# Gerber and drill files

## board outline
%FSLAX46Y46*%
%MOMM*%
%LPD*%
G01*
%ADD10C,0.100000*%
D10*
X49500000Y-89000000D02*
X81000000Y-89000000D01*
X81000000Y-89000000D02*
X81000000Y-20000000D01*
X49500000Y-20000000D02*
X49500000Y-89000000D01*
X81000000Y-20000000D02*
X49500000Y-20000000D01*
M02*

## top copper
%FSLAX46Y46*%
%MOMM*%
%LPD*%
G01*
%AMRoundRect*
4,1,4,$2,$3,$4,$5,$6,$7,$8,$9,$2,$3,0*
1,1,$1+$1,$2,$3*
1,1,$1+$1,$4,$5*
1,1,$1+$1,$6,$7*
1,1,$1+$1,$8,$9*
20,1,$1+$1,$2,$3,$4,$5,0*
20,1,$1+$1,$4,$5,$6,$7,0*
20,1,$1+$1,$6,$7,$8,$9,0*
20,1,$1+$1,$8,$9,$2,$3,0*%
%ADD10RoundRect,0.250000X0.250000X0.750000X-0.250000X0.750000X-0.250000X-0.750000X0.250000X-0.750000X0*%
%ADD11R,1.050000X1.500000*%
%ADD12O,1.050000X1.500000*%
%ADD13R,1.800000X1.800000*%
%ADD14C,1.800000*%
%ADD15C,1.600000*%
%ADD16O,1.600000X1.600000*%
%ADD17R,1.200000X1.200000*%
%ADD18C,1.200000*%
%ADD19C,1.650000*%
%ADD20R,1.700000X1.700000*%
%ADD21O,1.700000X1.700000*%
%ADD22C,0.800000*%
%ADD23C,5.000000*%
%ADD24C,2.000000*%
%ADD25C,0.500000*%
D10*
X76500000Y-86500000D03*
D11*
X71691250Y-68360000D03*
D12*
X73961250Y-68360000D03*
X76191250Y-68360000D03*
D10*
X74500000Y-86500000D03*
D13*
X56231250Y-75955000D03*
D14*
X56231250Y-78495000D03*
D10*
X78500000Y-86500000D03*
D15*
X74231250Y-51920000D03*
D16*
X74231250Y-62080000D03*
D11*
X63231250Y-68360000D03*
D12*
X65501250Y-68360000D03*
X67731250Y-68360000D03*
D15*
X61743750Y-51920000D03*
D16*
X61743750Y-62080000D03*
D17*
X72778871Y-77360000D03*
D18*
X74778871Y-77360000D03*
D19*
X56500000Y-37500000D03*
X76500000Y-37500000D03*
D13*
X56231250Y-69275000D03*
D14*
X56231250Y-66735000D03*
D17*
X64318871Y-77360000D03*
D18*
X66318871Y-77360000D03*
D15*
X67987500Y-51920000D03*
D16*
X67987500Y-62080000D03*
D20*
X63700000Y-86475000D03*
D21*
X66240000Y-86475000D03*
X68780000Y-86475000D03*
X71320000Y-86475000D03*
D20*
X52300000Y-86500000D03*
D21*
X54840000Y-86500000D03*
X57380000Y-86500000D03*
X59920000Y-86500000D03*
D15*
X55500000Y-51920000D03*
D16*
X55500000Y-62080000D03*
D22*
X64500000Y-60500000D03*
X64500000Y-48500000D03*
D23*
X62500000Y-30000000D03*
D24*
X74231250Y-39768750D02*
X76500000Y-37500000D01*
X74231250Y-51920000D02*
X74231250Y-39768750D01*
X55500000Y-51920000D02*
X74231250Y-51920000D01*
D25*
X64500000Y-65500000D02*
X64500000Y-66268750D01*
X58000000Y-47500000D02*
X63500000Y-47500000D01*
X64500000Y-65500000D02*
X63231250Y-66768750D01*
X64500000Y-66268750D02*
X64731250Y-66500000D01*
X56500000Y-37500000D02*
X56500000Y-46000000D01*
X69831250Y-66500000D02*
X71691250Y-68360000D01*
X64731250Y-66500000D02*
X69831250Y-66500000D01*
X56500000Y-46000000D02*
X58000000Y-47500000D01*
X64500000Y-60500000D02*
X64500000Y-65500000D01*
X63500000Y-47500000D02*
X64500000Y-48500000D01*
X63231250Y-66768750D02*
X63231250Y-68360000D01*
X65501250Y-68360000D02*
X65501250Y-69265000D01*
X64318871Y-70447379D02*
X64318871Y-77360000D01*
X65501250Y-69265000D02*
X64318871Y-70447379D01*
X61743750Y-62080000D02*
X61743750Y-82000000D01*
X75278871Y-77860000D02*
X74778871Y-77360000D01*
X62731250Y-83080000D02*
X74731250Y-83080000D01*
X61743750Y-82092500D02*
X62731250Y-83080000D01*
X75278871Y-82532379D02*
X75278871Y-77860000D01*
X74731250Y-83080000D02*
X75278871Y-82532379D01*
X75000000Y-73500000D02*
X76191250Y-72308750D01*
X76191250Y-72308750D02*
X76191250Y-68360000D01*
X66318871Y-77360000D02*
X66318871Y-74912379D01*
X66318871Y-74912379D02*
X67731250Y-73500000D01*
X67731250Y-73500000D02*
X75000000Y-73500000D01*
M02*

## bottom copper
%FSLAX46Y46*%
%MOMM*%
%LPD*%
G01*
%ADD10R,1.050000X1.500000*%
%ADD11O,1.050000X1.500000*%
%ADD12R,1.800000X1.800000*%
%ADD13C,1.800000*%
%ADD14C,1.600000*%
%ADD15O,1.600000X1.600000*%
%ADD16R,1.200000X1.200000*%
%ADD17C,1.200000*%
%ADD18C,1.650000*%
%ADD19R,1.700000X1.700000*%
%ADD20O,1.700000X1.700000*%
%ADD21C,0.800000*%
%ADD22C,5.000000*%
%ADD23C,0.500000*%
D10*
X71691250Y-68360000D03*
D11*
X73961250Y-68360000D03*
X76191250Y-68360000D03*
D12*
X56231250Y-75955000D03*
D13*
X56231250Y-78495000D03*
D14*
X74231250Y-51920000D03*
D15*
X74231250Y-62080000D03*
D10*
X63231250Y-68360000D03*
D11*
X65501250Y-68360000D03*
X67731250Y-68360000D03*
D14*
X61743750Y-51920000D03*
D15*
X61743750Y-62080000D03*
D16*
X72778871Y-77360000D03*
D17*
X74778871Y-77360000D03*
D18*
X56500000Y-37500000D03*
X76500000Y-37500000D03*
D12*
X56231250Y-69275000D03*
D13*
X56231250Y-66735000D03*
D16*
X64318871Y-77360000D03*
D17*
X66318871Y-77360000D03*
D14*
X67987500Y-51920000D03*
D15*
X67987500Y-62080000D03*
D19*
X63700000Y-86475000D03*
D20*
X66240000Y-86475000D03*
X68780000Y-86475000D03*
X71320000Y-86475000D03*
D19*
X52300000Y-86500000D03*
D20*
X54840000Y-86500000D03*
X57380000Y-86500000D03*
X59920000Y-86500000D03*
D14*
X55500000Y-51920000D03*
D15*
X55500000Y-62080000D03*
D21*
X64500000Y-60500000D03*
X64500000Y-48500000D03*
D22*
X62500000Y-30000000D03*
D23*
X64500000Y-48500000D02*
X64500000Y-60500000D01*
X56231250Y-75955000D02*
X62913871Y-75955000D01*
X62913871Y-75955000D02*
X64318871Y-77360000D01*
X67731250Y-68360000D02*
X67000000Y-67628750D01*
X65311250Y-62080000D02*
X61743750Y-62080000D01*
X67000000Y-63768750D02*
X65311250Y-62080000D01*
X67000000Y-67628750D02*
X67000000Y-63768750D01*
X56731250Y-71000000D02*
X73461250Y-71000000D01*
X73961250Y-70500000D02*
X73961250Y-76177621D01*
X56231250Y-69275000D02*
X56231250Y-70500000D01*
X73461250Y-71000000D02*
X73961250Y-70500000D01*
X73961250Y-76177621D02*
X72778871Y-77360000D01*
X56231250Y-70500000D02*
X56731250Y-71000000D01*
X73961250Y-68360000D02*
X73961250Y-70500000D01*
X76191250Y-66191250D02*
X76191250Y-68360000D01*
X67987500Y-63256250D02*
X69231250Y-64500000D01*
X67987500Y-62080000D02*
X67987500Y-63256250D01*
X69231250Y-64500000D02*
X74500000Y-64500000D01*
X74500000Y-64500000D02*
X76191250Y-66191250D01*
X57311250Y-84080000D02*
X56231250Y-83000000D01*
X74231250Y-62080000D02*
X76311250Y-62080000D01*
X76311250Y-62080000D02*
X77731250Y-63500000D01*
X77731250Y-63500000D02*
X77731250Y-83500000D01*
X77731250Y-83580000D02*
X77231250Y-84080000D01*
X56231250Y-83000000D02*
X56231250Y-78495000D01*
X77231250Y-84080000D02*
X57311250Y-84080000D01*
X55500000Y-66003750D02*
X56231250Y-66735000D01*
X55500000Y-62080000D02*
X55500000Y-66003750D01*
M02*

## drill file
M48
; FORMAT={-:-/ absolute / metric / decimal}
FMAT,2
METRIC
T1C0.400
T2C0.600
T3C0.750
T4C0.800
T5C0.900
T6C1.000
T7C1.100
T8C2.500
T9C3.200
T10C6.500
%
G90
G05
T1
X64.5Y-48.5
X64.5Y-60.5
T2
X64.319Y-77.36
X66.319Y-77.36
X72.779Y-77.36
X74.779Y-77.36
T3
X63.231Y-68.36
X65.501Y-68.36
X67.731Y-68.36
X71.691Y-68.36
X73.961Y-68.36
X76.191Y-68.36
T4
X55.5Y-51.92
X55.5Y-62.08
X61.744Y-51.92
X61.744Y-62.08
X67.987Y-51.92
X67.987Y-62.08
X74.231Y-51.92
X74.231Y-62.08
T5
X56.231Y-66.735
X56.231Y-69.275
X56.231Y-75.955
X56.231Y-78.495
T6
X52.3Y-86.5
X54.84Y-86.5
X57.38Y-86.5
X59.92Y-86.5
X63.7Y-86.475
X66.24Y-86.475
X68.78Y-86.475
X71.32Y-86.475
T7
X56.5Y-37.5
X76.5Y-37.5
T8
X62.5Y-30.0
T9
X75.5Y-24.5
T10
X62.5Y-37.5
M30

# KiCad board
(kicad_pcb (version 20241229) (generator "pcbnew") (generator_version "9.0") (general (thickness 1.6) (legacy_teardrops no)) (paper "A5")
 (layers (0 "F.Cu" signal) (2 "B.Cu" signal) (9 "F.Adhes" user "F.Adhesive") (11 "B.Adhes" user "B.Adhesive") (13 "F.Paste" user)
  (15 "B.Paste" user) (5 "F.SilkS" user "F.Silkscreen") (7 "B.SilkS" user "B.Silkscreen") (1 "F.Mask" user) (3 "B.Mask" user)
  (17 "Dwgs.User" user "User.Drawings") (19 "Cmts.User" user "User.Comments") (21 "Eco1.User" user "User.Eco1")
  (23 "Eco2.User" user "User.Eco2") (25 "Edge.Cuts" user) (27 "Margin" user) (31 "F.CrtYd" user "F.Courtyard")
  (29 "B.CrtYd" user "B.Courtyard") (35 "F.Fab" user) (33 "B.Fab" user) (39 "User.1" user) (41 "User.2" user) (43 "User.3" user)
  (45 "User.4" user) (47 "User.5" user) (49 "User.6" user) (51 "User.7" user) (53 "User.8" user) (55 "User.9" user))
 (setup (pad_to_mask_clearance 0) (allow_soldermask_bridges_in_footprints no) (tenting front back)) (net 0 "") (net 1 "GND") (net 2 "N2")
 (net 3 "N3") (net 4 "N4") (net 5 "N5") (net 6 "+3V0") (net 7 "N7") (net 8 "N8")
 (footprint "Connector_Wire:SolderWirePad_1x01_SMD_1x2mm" (layer "F.Cu") (at 76.5 86.5 180)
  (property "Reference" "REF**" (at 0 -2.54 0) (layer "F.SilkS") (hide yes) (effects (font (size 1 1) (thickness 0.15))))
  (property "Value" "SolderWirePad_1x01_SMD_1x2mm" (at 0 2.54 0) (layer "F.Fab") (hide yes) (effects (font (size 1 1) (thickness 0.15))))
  (pad "1" smd roundrect (at 0 0 180) (size 1 2) (layers "F.Cu" "F.Mask" "F.Paste") (roundrect_rratio 0.25)))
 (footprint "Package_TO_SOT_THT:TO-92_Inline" (layer "F.Cu") (at 72.69125 68.36)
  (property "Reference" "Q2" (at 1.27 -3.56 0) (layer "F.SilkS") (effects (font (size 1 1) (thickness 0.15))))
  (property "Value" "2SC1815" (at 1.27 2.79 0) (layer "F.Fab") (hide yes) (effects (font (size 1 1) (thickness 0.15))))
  (pad "1" thru_hole rect (at -1 0) (size 1.05 1.5) (drill 0.75) (layers "*.Cu" "*.Mask") (remove_unused_layers no) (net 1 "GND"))
  (pad "2" thru_hole oval (at 1.27 0) (size 1.05 1.5) (drill 0.75) (layers "*.Cu" "*.Mask") (remove_unused_layers no) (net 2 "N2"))
  (pad "3" thru_hole oval (at 3.5 0) (size 1.05 1.5) (drill 0.75) (layers "*.Cu" "*.Mask") (remove_unused_layers no) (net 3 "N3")))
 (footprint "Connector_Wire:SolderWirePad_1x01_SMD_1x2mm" (layer "F.Cu") (at 74.5 86.5 180)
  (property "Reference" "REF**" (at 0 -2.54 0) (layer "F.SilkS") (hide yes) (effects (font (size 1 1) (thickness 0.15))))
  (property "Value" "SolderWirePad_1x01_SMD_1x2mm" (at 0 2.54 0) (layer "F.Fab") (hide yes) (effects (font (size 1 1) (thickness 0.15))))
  (pad "1" smd roundrect (at 0 0 180) (size 1 2) (layers "F.Cu" "F.Mask" "F.Paste") (roundrect_rratio 0.25)))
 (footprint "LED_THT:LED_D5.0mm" (layer "F.Cu") (at 56.23125 75.955 -90)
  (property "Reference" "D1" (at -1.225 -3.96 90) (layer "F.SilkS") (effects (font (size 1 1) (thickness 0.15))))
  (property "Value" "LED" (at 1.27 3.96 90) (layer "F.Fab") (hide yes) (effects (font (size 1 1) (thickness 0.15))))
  (pad "1" thru_hole rect (at 0 0 270) (size 1.8 1.8) (drill 0.9) (layers "*.Cu" "*.Mask") (remove_unused_layers no) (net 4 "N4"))
  (pad "2" thru_hole circle (at 2.54 0 270) (size 1.8 1.8) (drill 0.9) (layers "*.Cu" "*.Mask") (remove_unused_layers no) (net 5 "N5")))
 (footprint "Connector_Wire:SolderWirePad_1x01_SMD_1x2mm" (layer "F.Cu") (at 78.5 86.5 180)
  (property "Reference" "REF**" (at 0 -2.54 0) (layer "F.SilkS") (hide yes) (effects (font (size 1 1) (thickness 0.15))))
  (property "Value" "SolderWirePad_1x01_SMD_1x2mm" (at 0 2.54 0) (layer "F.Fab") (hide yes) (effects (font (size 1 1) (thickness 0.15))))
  (pad "1" smd roundrect (at 0 0 180) (size 1 2) (layers "F.Cu" "F.Mask" "F.Paste") (roundrect_rratio 0.25)))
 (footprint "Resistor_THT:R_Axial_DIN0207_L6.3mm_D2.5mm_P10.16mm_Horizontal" (layer "F.Cu") (at 74.23125 51.92 -90)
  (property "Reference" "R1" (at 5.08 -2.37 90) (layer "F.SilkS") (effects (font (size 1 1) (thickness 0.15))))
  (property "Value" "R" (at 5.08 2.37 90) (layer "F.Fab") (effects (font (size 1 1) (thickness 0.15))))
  (pad "1" thru_hole circle (at 0 0 270) (size 1.6 1.6) (drill 0.8) (layers "*.Cu" "*.Mask") (remove_unused_layers no) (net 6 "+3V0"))
  (pad "2" thru_hole oval (at 10.16 0 270) (size 1.6 1.6) (drill 0.8) (layers "*.Cu" "*.Mask") (remove_unused_layers no) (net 5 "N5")))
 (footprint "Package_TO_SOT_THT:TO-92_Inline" (layer "F.Cu") (at 64.23125 68.36)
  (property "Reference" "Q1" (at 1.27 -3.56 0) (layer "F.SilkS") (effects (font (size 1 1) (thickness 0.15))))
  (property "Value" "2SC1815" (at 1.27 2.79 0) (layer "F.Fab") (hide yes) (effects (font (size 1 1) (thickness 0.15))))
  (pad "1" thru_hole rect (at -1 0) (size 1.05 1.5) (drill 0.75) (layers "*.Cu" "*.Mask") (remove_unused_layers no) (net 1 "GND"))
  (pad "2" thru_hole oval (at 1.27 0) (size 1.05 1.5) (drill 0.75) (layers "*.Cu" "*.Mask") (remove_unused_layers no) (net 4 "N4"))
  (pad "3" thru_hole oval (at 3.5 0) (size 1.05 1.5) (drill 0.75) (layers "*.Cu" "*.Mask") (remove_unused_layers no) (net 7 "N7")))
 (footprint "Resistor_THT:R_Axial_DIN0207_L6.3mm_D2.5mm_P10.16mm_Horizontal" (layer "F.Cu") (at 61.74375 51.92 -90)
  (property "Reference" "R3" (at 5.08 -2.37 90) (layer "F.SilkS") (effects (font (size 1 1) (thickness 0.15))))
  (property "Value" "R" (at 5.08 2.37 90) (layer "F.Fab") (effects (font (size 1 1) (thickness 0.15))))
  (pad "1" thru_hole circle (at 0 0 270) (size 1.6 1.6) (drill 0.8) (layers "*.Cu" "*.Mask") (remove_unused_layers no) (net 6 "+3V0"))
  (pad "2" thru_hole oval (at 10.16 0 270) (size 1.6 1.6) (drill 0.8) (layers "*.Cu" "*.Mask") (remove_unused_layers no) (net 7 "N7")))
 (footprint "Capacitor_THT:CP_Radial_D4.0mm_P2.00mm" (layer "F.Cu") (at 72.778871 77.36)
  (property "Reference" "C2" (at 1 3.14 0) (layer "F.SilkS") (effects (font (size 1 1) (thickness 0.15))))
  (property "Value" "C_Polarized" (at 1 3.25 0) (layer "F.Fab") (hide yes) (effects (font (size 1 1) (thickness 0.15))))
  (pad "1" thru_hole rect (at 0 0) (size 1.2 1.2) (drill 0.6) (layers "*.Cu" "*.Mask") (remove_unused_layers no) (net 2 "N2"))
  (pad "2" thru_hole circle (at 2 0) (size 1.2 1.2) (drill 0.6) (layers "*.Cu" "*.Mask") (remove_unused_layers no) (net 7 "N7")))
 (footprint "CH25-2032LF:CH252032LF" (layer "F.Cu") (at 56.5 37.5 90)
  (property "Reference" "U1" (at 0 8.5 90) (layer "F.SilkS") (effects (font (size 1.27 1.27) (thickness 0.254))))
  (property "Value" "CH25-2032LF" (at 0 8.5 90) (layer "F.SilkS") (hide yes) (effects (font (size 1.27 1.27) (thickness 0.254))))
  (pad "" np_thru_hole circle (at 0 6 90) (size 6.5 6.5) (drill 6.5) (layers "*.Cu" "*.Mask"))
  (pad "1" thru_hole circle (at 0 0 90) (size 1.65 1.65) (drill 1.1) (layers "*.Cu" "*.Mask") (remove_unused_layers no) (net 1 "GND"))
  (pad "2" thru_hole circle (at 0 20 90) (size 1.65 1.65) (drill 1.1) (layers "*.Cu" "*.Mask") (remove_unused_layers no) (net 6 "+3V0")))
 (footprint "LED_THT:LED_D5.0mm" (layer "F.Cu") (at 56.23125 69.275 90)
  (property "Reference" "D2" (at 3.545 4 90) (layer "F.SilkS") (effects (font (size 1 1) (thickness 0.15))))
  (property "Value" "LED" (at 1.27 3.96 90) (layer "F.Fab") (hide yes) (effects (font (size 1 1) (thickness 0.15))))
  (pad "1" thru_hole rect (at 0 0 90) (size 1.8 1.8) (drill 0.9) (layers "*.Cu" "*.Mask") (remove_unused_layers no) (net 2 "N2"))
  (pad "2" thru_hole circle (at 2.54 0 90) (size 1.8 1.8) (drill 0.9) (layers "*.Cu" "*.Mask") (remove_unused_layers no) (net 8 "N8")))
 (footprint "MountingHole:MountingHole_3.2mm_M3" (layer "F.Cu") (at 75.5 24.5)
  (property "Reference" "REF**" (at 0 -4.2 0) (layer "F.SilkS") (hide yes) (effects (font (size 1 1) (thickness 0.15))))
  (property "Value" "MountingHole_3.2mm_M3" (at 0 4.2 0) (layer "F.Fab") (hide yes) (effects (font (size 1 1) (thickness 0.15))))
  (pad "" np_thru_hole circle (at 0 0) (size 3.2 3.2) (drill 3.2) (layers "*.Cu" "*.Mask")))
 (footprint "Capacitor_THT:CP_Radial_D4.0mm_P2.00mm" (layer "F.Cu") (at 64.318871 77.36)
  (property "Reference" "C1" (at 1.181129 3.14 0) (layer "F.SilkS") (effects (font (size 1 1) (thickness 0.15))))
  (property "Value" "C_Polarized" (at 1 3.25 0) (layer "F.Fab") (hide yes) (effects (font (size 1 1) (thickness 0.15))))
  (pad "1" thru_hole rect (at 0 0) (size 1.2 1.2) (drill 0.6) (layers "*.Cu" "*.Mask") (remove_unused_layers no) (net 4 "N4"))
  (pad "2" thru_hole circle (at 2 0) (size 1.2 1.2) (drill 0.6) (layers "*.Cu" "*.Mask") (remove_unused_layers no) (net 3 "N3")))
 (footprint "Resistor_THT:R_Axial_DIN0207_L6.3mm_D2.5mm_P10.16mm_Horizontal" (layer "F.Cu") (at 67.9875 51.92 -90)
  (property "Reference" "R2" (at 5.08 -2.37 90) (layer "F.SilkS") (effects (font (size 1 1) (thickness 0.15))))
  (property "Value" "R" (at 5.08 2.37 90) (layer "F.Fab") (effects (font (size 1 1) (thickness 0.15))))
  (pad "1" thru_hole circle (at 0 0 270) (size 1.6 1.6) (drill 0.8) (layers "*.Cu" "*.Mask") (remove_unused_layers no) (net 6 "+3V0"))
  (pad "2" thru_hole oval (at 10.16 0 270) (size 1.6 1.6) (drill 0.8) (layers "*.Cu" "*.Mask") (remove_unused_layers no) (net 3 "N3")))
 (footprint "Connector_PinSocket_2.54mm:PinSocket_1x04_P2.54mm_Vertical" (layer "F.Cu") (at 63.7 86.475 90)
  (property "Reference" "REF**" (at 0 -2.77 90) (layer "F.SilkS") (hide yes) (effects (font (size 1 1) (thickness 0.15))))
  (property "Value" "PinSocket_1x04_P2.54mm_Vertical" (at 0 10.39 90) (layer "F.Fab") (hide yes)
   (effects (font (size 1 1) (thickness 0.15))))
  (pad "1" thru_hole rect (at 0 0 90) (size 1.7 1.7) (drill 1) (layers "*.Cu" "*.Mask") (remove_unused_layers no))
  (pad "2" thru_hole oval (at 0 2.54 90) (size 1.7 1.7) (drill 1) (layers "*.Cu" "*.Mask") (remove_unused_layers no))
  (pad "3" thru_hole oval (at 0 5.08 90) (size 1.7 1.7) (drill 1) (layers "*.Cu" "*.Mask") (remove_unused_layers no))
  (pad "4" thru_hole oval (at 0 7.62 90) (size 1.7 1.7) (drill 1) (layers "*.Cu" "*.Mask") (remove_unused_layers no)))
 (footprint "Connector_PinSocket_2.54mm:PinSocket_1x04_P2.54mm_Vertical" (layer "F.Cu") (at 52.3 86.5 90)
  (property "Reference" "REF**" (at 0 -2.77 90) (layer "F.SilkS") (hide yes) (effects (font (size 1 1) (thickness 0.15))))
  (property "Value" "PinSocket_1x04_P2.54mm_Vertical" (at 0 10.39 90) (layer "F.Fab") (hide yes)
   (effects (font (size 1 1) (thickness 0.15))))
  (pad "1" thru_hole rect (at 0 0 90) (size 1.7 1.7) (drill 1) (layers "*.Cu" "*.Mask") (remove_unused_layers no))
  (pad "2" thru_hole oval (at 0 2.54 90) (size 1.7 1.7) (drill 1) (layers "*.Cu" "*.Mask") (remove_unused_layers no))
  (pad "3" thru_hole oval (at 0 5.08 90) (size 1.7 1.7) (drill 1) (layers "*.Cu" "*.Mask") (remove_unused_layers no))
  (pad "4" thru_hole oval (at 0 7.62 90) (size 1.7 1.7) (drill 1) (layers "*.Cu" "*.Mask") (remove_unused_layers no)))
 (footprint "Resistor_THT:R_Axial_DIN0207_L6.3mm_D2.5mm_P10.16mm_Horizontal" (layer "F.Cu") (at 55.5 51.92 -90)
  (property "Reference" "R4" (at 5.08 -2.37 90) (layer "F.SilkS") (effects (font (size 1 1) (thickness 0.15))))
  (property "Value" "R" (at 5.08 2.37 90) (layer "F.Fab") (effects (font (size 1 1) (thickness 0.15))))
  (pad "1" thru_hole circle (at 0 0 270) (size 1.6 1.6) (drill 0.8) (layers "*.Cu" "*.Mask") (remove_unused_layers no) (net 6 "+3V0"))
  (pad "2" thru_hole oval (at 10.16 0 270) (size 1.6 1.6) (drill 0.8) (layers "*.Cu" "*.Mask") (remove_unused_layers no) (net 8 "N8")))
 (gr_line (start 49.5 89) (end 81 89) (stroke (width 0.1) (type default)) (layer "Edge.Cuts"))
 (gr_line (start 81 89) (end 81 20) (stroke (width 0.1) (type default)) (layer "Edge.Cuts"))
 (gr_line (start 49.5 20) (end 49.5 89) (stroke (width 0.1) (type default)) (layer "Edge.Cuts"))
 (gr_line (start 81 20) (end 49.5 20) (stroke (width 0.1) (type default)) (layer "Edge.Cuts"))
 (segment (start 74.23125 39.76875) (end 76.5 37.5) (width 2) (layer "F.Cu") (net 6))
 (segment (start 74.23125 51.92) (end 74.23125 39.76875) (width 2) (layer "F.Cu") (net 6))
 (segment (start 55.5 51.92) (end 74.23125 51.92) (width 2) (layer "F.Cu") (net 6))
 (segment (start 64.5 65.5) (end 64.5 66.26875) (width 0.5) (layer "F.Cu") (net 1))
 (segment (start 58 47.5) (end 63.5 47.5) (width 0.5) (layer "F.Cu") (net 1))
 (segment (start 64.5 65.5) (end 63.23125 66.76875) (width 0.5) (layer "F.Cu") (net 1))
 (segment (start 64.5 66.26875) (end 64.73125 66.5) (width 0.5) (layer "F.Cu") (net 1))
 (segment (start 56.5 37.5) (end 56.5 46) (width 0.5) (layer "F.Cu") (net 1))
 (segment (start 69.83125 66.5) (end 71.69125 68.36) (width 0.5) (layer "F.Cu") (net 1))
 (segment (start 64.73125 66.5) (end 69.83125 66.5) (width 0.5) (layer "F.Cu") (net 1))
 (segment (start 56.5 46) (end 58 47.5) (width 0.5) (layer "F.Cu") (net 1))
 (segment (start 64.5 60.5) (end 64.5 65.5) (width 0.5) (layer "F.Cu") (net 1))
 (segment (start 63.5 47.5) (end 64.5 48.5) (width 0.5) (layer "F.Cu") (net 1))
 (segment (start 63.23125 66.76875) (end 63.23125 68.36) (width 0.5) (layer "F.Cu") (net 1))
 (via (at 64.5 60.5) (size 0.8) (drill 0.4) (layers "F.Cu" "B.Cu") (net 1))
 (via (at 64.5 48.5) (size 0.8) (drill 0.4) (layers "F.Cu" "B.Cu") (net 1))
 (via (at 62.5 30) (size 5) (drill 2.5) (layers "F.Cu" "B.Cu") (free yes) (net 1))
 (segment (start 64.5 48.5) (end 64.5 60.5) (width 0.5) (layer "B.Cu") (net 1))
 (segment (start 65.50125 68.36) (end 65.50125 69.265) (width 0.5) (layer "F.Cu") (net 4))
 (segment (start 64.318871 70.447379) (end 64.318871 77.36) (width 0.5) (layer "F.Cu") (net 4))
 (segment (start 65.50125 69.265) (end 64.318871 70.447379) (width 0.5) (layer "F.Cu") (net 4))
 (segment (start 56.23125 75.955) (end 62.913871 75.955) (width 0.5) (layer "B.Cu") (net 4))
 (segment (start 62.913871 75.955) (end 64.318871 77.36) (width 0.5) (layer "B.Cu") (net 4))
 (segment (start 61.74375 62.08) (end 61.74375 82) (width 0.5) (layer "F.Cu") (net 7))
 (segment (start 75.278871 77.86) (end 74.778871 77.36) (width 0.5) (layer "F.Cu") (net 7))
 (segment (start 62.73125 83.08) (end 74.73125 83.08) (width 0.5) (layer "F.Cu") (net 7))
 (segment (start 61.74375 82.0925) (end 62.73125 83.08) (width 0.5) (layer "F.Cu") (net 7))
 (segment (start 75.278871 82.532379) (end 75.278871 77.86) (width 0.5) (layer "F.Cu") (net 7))
 (segment (start 74.73125 83.08) (end 75.278871 82.532379) (width 0.5) (layer "F.Cu") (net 7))
 (segment (start 67.73125 68.36) (end 67 67.62875) (width 0.5) (layer "B.Cu") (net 7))
 (segment (start 65.31125 62.08) (end 61.74375 62.08) (width 0.5) (layer "B.Cu") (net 7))
 (segment (start 67 63.76875) (end 65.31125 62.08) (width 0.5) (layer "B.Cu") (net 7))
 (segment (start 67 67.62875) (end 67 63.76875) (width 0.5) (layer "B.Cu") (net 7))
 (segment (start 56.73125 71) (end 73.46125 71) (width 0.5) (layer "B.Cu") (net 2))
 (segment (start 73.96125 70.5) (end 73.96125 76.177621) (width 0.5) (layer "B.Cu") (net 2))
 (segment (start 56.23125 69.275) (end 56.23125 70.5) (width 0.5) (layer "B.Cu") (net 2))
 (segment (start 73.46125 71) (end 73.96125 70.5) (width 0.5) (layer "B.Cu") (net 2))
 (segment (start 73.96125 76.177621) (end 72.778871 77.36) (width 0.5) (layer "B.Cu") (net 2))
 (segment (start 56.23125 70.5) (end 56.73125 71) (width 0.5) (layer "B.Cu") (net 2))
 (segment (start 73.96125 68.36) (end 73.96125 70.5) (width 0.5) (layer "B.Cu") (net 2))
 (segment (start 75 73.5) (end 76.19125 72.30875) (width 0.5) (layer "F.Cu") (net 3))
 (segment (start 76.19125 72.30875) (end 76.19125 68.36) (width 0.5) (layer "F.Cu") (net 3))
 (segment (start 66.318871 77.36) (end 66.318871 74.912379) (width 0.5) (layer "F.Cu") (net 3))
 (segment (start 66.318871 74.912379) (end 67.73125 73.5) (width 0.5) (layer "F.Cu") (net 3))
 (segment (start 67.73125 73.5) (end 75 73.5) (width 0.5) (layer "F.Cu") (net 3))
 (segment (start 76.19125 66.19125) (end 76.19125 68.36) (width 0.5) (layer "B.Cu") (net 3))
 (segment (start 67.9875 63.25625) (end 69.23125 64.5) (width 0.5) (layer "B.Cu") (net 3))
 (segment (start 67.9875 62.08) (end 67.9875 63.25625) (width 0.5) (layer "B.Cu") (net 3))
 (segment (start 69.23125 64.5) (end 74.5 64.5) (width 0.5) (layer "B.Cu") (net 3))
 (segment (start 74.5 64.5) (end 76.19125 66.19125) (width 0.5) (layer "B.Cu") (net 3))
 (segment (start 57.31125 84.08) (end 56.23125 83) (width 0.5) (layer "B.Cu") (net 5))
 (segment (start 74.23125 62.08) (end 76.31125 62.08) (width 0.5) (layer "B.Cu") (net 5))
 (segment (start 76.31125 62.08) (end 77.73125 63.5) (width 0.5) (layer "B.Cu") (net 5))
 (segment (start 77.73125 63.5) (end 77.73125 83.5) (width 0.5) (layer "B.Cu") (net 5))
 (segment (start 77.73125 83.58) (end 77.23125 84.08) (width 0.5) (layer "B.Cu") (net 5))
 (segment (start 56.23125 83) (end 56.23125 78.495) (width 0.5) (layer "B.Cu") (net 5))
 (segment (start 77.23125 84.08) (end 57.31125 84.08) (width 0.5) (layer "B.Cu") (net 5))
 (segment (start 55.5 66.00375) (end 56.23125 66.735) (width 0.5) (layer "B.Cu") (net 8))
 (segment (start 55.5 62.08) (end 55.5 66.00375) (width 0.5) (layer "B.Cu") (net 8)))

